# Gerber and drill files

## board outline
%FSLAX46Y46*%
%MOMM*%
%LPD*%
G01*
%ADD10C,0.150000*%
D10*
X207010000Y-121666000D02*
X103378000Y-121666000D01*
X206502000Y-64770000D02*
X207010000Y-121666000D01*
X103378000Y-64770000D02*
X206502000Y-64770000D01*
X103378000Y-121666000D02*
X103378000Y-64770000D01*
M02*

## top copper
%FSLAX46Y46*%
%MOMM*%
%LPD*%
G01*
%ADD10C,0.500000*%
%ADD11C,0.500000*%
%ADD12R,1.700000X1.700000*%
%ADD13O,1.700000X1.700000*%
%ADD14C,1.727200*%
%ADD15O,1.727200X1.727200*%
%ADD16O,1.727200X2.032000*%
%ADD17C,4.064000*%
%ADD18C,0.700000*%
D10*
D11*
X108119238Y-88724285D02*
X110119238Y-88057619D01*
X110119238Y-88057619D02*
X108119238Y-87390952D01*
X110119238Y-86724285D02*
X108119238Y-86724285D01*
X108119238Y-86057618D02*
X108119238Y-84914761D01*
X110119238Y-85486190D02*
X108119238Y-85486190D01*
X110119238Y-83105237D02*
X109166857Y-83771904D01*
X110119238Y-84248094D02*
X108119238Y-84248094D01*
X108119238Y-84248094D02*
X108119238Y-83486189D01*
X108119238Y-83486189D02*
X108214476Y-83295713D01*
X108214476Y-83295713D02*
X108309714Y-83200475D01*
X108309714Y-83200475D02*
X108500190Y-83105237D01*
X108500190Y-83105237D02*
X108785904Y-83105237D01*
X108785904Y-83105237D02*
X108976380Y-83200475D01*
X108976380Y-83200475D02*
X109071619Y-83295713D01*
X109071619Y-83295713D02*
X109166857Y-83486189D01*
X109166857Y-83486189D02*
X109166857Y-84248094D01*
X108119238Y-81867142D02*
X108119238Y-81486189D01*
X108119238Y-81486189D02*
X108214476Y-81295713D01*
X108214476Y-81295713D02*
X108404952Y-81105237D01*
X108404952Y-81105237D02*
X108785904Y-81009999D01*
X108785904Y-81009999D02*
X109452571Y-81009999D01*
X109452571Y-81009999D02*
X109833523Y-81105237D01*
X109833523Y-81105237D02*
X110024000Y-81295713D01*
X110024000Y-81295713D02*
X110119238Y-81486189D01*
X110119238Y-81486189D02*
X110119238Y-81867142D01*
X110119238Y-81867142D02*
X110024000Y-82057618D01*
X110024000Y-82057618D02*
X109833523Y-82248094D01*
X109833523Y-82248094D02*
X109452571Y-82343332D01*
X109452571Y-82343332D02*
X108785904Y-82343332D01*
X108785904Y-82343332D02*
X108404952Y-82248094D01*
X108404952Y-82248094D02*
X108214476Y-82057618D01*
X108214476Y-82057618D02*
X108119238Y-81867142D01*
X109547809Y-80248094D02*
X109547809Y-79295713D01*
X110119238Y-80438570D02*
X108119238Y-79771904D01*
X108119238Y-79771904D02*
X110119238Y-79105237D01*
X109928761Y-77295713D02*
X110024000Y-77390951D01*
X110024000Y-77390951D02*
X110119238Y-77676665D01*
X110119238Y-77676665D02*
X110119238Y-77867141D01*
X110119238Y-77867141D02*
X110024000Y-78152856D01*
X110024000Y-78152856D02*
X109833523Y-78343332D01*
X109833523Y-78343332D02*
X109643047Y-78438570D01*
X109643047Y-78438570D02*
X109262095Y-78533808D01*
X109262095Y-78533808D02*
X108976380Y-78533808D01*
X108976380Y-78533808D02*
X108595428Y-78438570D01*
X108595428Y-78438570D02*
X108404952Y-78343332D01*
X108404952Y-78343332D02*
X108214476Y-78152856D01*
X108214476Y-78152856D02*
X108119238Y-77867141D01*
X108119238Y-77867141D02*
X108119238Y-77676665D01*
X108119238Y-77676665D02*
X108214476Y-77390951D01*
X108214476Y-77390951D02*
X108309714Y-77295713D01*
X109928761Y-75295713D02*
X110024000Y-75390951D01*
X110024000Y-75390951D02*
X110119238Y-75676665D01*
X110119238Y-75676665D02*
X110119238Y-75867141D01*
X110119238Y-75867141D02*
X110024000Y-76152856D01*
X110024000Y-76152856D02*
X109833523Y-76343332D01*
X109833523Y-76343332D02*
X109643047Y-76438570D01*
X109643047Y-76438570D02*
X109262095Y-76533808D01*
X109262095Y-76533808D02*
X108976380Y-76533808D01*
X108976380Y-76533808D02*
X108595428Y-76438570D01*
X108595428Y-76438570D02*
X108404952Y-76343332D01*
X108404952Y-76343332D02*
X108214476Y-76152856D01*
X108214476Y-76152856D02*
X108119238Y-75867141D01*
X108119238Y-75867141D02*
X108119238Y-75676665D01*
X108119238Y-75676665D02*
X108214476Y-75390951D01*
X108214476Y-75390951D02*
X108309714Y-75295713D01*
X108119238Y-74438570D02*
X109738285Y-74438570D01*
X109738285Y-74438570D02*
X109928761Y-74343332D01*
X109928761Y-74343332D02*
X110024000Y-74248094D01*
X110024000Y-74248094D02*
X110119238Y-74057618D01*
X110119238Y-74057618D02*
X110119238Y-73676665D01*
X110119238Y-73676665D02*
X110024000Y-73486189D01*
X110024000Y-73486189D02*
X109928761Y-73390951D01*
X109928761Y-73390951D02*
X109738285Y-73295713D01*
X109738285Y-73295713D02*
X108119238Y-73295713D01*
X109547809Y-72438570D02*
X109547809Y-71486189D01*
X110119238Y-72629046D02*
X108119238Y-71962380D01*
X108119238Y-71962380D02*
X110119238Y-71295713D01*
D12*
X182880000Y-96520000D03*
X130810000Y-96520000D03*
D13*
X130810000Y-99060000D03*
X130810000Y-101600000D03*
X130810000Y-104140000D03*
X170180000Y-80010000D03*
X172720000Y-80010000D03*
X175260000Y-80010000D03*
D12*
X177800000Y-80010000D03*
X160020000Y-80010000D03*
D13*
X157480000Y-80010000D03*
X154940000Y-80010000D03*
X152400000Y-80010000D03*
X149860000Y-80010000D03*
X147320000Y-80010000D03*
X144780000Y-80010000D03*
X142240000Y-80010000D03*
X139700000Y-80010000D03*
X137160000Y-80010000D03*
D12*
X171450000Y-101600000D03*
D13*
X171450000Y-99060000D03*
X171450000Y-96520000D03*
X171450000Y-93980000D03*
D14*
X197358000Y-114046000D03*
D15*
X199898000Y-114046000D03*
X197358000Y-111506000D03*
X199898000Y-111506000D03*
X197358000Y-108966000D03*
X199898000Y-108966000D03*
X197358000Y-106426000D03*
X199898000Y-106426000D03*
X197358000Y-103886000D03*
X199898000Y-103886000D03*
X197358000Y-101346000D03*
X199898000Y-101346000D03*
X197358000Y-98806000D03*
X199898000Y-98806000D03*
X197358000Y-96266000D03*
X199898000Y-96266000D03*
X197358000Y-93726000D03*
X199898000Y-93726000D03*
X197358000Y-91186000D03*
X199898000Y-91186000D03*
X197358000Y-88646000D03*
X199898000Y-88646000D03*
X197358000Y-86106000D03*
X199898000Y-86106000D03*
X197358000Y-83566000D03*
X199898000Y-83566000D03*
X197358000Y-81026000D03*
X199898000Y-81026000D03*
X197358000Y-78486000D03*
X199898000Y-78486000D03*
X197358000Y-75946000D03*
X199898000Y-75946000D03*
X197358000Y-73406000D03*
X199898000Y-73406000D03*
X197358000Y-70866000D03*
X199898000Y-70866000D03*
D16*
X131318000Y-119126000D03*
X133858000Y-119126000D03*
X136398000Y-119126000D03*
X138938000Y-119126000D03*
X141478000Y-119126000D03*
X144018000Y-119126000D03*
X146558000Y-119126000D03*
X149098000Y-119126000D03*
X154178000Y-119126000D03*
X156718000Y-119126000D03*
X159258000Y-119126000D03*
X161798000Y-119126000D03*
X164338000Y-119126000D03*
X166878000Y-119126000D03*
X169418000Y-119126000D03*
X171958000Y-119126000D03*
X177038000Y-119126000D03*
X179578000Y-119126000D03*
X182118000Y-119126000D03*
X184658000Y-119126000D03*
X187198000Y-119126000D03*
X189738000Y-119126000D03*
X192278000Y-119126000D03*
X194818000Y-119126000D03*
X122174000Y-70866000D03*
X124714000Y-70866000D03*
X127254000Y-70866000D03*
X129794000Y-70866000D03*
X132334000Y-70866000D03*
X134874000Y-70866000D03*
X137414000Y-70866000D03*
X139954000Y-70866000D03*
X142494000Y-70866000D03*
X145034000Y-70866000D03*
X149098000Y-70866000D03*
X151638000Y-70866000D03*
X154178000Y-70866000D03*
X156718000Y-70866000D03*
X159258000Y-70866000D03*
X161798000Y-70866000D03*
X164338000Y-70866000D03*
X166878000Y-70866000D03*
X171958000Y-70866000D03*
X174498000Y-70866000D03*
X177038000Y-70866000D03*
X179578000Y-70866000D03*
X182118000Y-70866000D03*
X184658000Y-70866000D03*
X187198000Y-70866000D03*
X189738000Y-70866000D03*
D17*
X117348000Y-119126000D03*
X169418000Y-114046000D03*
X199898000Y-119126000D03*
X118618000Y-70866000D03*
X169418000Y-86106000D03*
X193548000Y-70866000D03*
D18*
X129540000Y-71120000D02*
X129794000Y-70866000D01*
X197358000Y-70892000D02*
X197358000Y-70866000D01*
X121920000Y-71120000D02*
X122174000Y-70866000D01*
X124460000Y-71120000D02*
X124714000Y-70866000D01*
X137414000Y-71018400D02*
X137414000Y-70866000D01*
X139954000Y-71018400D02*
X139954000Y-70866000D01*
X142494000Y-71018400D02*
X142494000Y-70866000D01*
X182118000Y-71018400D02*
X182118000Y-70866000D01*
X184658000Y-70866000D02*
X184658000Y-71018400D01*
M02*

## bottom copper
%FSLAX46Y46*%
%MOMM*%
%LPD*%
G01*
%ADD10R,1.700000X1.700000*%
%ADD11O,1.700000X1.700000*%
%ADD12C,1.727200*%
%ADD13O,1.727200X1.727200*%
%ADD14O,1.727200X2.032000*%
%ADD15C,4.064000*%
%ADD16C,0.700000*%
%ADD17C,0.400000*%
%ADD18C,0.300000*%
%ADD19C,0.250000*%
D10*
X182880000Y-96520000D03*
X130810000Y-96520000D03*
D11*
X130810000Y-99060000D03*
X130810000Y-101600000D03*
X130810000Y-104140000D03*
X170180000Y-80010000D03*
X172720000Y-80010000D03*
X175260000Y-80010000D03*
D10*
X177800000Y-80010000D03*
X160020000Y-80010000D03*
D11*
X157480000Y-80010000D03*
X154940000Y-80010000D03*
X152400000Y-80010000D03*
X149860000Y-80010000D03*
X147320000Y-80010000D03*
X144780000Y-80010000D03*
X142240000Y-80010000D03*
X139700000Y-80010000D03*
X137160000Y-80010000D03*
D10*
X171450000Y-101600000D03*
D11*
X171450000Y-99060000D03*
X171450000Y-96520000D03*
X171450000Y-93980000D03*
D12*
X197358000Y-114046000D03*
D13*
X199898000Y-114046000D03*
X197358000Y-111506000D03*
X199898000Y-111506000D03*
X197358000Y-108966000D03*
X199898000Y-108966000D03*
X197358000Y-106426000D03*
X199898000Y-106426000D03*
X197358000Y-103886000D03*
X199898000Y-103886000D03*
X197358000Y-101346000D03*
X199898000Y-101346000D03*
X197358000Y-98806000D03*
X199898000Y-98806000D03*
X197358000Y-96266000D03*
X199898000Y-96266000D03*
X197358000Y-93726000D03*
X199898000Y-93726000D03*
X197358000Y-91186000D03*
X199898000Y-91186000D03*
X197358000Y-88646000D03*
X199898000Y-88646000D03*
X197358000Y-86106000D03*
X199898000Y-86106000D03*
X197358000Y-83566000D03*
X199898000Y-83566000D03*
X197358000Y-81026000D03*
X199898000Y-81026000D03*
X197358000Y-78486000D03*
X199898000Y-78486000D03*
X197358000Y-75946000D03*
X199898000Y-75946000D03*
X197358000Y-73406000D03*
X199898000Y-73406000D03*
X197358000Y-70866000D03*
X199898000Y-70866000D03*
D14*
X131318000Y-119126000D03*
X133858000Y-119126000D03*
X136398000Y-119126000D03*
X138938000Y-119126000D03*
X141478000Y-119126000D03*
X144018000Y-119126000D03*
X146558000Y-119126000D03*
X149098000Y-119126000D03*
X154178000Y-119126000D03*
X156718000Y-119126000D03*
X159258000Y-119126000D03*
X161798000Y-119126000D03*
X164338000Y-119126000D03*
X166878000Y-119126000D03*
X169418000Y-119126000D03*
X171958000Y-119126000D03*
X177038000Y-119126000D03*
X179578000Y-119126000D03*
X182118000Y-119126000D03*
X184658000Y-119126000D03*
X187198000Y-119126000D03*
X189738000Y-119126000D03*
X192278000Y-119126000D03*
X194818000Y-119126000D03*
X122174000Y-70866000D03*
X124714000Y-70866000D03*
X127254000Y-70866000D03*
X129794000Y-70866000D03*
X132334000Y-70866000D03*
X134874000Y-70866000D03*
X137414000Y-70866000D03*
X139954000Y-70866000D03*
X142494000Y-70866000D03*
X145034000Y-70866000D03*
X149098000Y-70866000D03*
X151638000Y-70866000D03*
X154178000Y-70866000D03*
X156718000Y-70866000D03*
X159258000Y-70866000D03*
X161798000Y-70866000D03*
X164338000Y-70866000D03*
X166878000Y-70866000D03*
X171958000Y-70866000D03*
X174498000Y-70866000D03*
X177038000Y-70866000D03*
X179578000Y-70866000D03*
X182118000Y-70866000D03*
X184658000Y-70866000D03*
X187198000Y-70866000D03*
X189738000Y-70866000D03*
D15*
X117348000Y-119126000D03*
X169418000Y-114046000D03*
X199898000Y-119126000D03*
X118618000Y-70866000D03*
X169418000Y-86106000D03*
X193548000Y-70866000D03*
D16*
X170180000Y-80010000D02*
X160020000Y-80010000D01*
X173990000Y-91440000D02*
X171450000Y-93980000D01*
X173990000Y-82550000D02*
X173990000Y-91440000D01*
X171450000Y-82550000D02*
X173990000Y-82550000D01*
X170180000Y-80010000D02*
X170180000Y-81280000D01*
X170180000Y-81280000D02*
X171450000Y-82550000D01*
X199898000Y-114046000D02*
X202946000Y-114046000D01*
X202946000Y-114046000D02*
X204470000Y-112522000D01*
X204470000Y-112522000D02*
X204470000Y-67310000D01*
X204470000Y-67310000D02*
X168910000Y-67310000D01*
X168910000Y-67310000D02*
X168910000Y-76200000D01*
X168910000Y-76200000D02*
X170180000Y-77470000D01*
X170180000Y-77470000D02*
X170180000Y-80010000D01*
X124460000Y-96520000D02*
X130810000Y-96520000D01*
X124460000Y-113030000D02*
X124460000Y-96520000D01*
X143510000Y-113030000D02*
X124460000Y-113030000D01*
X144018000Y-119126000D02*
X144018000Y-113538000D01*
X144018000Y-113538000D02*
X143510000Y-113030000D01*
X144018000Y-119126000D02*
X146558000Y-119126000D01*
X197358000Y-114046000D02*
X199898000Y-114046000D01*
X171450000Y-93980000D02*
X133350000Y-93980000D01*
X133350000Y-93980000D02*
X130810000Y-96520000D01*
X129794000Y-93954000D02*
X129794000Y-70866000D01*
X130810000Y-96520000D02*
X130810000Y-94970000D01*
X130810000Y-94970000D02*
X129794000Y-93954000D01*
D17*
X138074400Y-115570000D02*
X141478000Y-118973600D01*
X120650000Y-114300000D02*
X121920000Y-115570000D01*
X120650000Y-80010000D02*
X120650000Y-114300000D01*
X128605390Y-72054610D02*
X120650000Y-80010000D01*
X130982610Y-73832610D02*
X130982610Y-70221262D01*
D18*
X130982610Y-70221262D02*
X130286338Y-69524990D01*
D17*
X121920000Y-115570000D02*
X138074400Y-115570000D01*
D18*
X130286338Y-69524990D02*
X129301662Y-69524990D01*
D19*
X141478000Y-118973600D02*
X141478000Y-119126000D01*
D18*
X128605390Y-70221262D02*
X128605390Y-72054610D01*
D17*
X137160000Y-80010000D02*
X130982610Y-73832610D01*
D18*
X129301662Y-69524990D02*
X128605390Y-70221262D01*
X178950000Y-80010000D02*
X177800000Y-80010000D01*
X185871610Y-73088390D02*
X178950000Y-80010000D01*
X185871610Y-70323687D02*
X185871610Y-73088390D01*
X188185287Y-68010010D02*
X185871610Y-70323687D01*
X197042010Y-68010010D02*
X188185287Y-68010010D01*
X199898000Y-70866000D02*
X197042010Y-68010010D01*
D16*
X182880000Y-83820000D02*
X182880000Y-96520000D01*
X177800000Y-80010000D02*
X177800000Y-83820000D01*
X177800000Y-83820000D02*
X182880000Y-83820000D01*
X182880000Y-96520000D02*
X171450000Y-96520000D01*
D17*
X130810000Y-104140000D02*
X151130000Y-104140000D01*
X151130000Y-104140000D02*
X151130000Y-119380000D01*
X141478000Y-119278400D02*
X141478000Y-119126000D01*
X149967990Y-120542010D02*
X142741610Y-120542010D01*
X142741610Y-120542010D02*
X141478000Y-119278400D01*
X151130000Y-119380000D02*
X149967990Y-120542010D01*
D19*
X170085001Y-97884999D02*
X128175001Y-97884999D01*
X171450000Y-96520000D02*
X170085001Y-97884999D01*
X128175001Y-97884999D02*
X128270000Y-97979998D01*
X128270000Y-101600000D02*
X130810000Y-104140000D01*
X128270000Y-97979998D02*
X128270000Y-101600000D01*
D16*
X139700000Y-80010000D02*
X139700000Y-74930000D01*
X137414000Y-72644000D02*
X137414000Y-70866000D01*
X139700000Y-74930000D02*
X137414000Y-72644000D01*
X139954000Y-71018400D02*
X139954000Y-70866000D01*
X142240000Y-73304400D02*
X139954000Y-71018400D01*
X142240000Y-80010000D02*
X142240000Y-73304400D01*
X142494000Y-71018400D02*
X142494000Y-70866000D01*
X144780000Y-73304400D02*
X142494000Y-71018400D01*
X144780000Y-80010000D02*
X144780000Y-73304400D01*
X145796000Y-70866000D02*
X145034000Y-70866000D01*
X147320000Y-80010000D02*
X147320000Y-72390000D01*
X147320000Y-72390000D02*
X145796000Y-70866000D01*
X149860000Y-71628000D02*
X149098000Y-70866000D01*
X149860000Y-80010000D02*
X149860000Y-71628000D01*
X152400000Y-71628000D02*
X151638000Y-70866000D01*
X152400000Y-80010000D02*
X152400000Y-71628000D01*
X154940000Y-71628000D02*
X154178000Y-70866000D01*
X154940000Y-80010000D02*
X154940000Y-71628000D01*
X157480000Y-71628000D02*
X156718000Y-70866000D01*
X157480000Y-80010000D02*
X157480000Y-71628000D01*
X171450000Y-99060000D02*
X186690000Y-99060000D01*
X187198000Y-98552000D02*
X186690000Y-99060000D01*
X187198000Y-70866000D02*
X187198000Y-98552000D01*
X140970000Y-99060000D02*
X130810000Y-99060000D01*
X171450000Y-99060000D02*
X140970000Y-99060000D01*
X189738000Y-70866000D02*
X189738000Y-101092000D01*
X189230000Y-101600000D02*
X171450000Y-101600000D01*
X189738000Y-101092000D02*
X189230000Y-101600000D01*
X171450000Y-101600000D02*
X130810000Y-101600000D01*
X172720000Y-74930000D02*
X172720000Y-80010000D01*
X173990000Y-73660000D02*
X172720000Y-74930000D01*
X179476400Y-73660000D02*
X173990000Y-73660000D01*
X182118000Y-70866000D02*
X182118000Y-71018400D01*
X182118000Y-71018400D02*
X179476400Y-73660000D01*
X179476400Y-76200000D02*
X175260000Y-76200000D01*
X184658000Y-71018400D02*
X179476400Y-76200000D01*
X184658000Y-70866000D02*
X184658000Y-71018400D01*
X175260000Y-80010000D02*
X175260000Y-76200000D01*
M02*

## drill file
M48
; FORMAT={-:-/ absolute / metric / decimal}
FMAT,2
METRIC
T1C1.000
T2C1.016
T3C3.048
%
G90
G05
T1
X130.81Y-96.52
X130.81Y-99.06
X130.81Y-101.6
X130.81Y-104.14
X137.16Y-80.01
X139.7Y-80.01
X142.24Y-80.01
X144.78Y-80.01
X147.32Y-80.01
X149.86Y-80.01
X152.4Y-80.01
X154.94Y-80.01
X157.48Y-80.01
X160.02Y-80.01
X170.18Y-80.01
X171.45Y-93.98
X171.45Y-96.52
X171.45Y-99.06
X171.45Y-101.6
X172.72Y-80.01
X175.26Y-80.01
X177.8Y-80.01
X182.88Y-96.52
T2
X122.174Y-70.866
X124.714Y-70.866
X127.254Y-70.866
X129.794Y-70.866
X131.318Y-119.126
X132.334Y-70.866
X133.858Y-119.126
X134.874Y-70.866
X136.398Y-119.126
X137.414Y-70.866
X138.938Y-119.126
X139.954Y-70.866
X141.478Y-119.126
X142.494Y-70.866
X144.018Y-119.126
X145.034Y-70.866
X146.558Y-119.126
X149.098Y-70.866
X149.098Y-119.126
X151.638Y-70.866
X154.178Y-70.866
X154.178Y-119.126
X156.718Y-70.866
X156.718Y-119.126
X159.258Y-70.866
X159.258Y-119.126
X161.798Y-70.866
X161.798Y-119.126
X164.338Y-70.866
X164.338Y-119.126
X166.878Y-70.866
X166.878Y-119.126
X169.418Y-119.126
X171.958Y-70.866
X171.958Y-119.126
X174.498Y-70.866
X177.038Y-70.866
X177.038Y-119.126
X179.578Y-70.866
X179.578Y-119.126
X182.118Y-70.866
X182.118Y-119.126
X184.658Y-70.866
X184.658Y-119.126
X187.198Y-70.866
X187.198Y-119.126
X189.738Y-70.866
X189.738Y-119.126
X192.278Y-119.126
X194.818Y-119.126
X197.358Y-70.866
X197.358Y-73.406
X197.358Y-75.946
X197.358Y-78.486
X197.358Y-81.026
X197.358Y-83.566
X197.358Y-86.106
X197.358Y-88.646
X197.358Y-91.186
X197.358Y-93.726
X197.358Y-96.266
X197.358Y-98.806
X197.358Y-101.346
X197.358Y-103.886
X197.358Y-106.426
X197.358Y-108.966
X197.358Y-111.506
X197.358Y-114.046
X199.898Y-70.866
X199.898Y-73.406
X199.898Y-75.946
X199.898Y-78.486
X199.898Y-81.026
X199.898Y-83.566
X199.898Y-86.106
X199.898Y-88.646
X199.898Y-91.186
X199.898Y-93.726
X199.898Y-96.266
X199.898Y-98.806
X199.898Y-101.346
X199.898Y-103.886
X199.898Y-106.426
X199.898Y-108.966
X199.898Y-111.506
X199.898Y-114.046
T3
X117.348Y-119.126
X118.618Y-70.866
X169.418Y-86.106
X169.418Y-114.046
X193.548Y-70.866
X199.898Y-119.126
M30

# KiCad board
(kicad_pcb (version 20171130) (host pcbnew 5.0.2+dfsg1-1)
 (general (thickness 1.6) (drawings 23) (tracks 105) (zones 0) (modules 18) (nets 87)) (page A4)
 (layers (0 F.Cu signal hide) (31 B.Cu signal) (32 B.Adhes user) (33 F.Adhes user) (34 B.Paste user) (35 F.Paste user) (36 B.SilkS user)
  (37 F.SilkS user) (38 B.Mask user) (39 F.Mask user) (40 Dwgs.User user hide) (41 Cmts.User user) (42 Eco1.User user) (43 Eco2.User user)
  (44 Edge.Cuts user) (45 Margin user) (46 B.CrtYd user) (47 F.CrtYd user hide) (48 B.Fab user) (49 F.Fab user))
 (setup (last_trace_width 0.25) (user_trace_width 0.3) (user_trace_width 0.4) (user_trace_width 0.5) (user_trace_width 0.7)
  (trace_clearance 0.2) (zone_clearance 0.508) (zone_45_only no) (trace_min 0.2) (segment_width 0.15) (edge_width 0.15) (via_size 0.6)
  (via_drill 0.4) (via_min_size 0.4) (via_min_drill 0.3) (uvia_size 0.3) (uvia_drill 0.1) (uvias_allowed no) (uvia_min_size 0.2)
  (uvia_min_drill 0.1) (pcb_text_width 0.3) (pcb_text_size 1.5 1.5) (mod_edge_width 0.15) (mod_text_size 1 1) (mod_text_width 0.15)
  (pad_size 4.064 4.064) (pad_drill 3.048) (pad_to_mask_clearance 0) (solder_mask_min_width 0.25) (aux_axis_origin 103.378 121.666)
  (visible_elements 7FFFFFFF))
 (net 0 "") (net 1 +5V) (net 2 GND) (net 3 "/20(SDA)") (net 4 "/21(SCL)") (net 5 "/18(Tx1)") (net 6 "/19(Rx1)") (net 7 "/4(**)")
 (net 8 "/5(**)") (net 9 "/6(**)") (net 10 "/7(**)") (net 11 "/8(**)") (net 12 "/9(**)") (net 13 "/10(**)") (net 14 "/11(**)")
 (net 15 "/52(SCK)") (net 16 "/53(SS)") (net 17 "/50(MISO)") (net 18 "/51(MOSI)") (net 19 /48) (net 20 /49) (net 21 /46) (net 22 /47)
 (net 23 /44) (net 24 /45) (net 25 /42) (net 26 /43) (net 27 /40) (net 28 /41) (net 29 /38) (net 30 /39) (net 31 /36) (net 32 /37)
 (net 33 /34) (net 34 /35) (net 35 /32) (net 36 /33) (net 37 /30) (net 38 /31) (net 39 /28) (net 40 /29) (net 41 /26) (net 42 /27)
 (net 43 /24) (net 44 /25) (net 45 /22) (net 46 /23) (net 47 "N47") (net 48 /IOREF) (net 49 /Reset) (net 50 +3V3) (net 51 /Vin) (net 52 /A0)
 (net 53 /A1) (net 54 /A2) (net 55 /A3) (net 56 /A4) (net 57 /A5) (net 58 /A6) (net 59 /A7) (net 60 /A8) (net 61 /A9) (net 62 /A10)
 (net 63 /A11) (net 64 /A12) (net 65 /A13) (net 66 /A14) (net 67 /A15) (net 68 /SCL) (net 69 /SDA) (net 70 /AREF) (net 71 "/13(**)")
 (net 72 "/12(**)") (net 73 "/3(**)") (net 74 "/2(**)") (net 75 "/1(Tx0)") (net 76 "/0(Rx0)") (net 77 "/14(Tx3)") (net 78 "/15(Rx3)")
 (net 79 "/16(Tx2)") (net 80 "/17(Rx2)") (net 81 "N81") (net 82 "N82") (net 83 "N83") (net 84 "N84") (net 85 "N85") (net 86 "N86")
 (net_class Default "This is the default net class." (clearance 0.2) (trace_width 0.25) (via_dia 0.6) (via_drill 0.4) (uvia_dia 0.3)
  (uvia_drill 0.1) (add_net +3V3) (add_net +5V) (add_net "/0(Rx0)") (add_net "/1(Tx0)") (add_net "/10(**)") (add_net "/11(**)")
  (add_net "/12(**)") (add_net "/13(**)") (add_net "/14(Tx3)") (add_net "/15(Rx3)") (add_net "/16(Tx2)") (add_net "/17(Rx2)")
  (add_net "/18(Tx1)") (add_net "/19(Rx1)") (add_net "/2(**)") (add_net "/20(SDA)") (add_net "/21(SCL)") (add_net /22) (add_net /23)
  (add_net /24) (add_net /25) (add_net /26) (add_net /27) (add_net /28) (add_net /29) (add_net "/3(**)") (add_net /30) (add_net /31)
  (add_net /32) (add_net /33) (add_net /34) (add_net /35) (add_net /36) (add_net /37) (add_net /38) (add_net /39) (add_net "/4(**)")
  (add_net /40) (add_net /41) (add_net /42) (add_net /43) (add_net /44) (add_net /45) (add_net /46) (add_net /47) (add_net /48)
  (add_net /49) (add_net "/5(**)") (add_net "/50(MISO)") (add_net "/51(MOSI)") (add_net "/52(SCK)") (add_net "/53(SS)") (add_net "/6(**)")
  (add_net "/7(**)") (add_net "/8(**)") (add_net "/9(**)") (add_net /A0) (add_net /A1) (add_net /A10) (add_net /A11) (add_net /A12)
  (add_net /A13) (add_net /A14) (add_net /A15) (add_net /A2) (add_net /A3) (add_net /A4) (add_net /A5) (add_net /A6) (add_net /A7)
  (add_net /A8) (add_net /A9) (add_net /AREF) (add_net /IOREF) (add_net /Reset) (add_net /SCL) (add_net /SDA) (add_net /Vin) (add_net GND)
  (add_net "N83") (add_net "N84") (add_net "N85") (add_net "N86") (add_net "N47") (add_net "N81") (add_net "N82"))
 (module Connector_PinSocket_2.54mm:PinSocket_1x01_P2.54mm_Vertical (layer F.Cu) (at 182.88 96.52)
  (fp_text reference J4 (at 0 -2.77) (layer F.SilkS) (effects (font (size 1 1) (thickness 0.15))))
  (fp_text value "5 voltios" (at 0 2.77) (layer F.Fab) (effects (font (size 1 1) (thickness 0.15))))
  (pad 1 thru_hole rect (at 0 0) (size 1.7 1.7) (drill 1) (layers *.Cu *.Mask) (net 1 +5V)))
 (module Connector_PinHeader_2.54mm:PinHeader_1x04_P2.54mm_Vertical (layer F.Cu) (at 130.81 96.52)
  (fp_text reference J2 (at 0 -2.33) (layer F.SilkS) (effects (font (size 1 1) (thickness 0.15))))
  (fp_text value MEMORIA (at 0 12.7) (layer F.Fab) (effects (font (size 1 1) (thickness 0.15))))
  (pad 1 thru_hole rect (at 0 0) (size 1.7 1.7) (drill 1) (layers *.Cu *.Mask) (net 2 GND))
  (pad 2 thru_hole oval (at 0 2.54) (size 1.7 1.7) (drill 1) (layers *.Cu *.Mask) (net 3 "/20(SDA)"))
  (pad 3 thru_hole oval (at 0 5.08) (size 1.7 1.7) (drill 1) (layers *.Cu *.Mask) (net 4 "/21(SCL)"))
  (pad 4 thru_hole oval (at 0 7.62) (size 1.7 1.7) (drill 1) (layers *.Cu *.Mask) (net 1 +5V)))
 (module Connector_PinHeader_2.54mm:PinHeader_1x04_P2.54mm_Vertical (layer F.Cu) (at 177.8 80.01 270)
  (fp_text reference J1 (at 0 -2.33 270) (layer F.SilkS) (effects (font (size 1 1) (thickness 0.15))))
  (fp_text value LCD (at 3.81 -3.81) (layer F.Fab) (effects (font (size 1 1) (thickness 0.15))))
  (pad 4 thru_hole oval (at 0 7.62 270) (size 1.7 1.7) (drill 1) (layers *.Cu *.Mask) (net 2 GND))
  (pad 3 thru_hole oval (at 0 5.08 270) (size 1.7 1.7) (drill 1) (layers *.Cu *.Mask) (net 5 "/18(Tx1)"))
  (pad 2 thru_hole oval (at 0 2.54 270) (size 1.7 1.7) (drill 1) (layers *.Cu *.Mask) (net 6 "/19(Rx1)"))
  (pad 1 thru_hole rect (at 0 0 270) (size 1.7 1.7) (drill 1) (layers *.Cu *.Mask) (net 1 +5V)))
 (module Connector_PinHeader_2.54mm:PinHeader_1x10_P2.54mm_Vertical (layer F.Cu) (at 160.02 80.01 270)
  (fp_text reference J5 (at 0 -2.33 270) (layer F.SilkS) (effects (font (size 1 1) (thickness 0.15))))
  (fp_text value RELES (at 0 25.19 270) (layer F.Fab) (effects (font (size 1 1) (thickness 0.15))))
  (pad 1 thru_hole rect (at 0 0 270) (size 1.7 1.7) (drill 1) (layers *.Cu *.Mask) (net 2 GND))
  (pad 2 thru_hole oval (at 0 2.54 270) (size 1.7 1.7) (drill 1) (layers *.Cu *.Mask) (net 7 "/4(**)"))
  (pad 3 thru_hole oval (at 0 5.08 270) (size 1.7 1.7) (drill 1) (layers *.Cu *.Mask) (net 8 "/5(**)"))
  (pad 4 thru_hole oval (at 0 7.62 270) (size 1.7 1.7) (drill 1) (layers *.Cu *.Mask) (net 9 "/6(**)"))
  (pad 5 thru_hole oval (at 0 10.16 270) (size 1.7 1.7) (drill 1) (layers *.Cu *.Mask) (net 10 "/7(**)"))
  (pad 6 thru_hole oval (at 0 12.7 270) (size 1.7 1.7) (drill 1) (layers *.Cu *.Mask) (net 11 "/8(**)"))
  (pad 7 thru_hole oval (at 0 15.24 270) (size 1.7 1.7) (drill 1) (layers *.Cu *.Mask) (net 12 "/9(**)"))
  (pad 8 thru_hole oval (at 0 17.78 270) (size 1.7 1.7) (drill 1) (layers *.Cu *.Mask) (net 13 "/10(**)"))
  (pad 9 thru_hole oval (at 0 20.32 270) (size 1.7 1.7) (drill 1) (layers *.Cu *.Mask) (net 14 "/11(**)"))
  (pad 10 thru_hole oval (at 0 22.86 270) (size 1.7 1.7) (drill 1) (layers *.Cu *.Mask) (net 1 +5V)))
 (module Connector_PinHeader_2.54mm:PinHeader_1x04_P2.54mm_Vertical (layer F.Cu) (at 171.45 101.6 180)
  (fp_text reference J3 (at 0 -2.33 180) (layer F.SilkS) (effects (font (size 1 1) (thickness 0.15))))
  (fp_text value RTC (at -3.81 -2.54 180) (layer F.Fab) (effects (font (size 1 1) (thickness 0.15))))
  (pad 1 thru_hole rect (at 0 0 180) (size 1.7 1.7) (drill 1) (layers *.Cu *.Mask) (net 4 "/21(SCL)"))
  (pad 2 thru_hole oval (at 0 2.54 180) (size 1.7 1.7) (drill 1) (layers *.Cu *.Mask) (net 3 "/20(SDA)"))
  (pad 3 thru_hole oval (at 0 5.08 180) (size 1.7 1.7) (drill 1) (layers *.Cu *.Mask) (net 1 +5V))
  (pad 4 thru_hole oval (at 0 7.62 180) (size 1.7 1.7) (drill 1) (layers *.Cu *.Mask) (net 2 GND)))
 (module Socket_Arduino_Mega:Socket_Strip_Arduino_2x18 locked (layer F.Cu) (at 197.358 114.046 90)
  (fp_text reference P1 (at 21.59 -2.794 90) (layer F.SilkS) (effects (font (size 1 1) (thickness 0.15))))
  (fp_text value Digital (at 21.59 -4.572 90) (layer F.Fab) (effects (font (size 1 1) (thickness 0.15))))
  (pad 1 thru_hole circle (at 0 0 90) (size 1.7272 1.7272) (drill 1.016) (layers *.Cu *.Mask F.SilkS) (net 2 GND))
  (pad 2 thru_hole oval (at 0 2.54 90) (size 1.7272 1.7272) (drill 1.016) (layers *.Cu *.Mask F.SilkS) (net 2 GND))
  (pad 3 thru_hole oval (at 2.54 0 90) (size 1.7272 1.7272) (drill 1.016) (layers *.Cu *.Mask F.SilkS) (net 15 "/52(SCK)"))
  (pad 4 thru_hole oval (at 2.54 2.54 90) (size 1.7272 1.7272) (drill 1.016) (layers *.Cu *.Mask F.SilkS) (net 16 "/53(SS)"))
  (pad 5 thru_hole oval (at 5.08 0 90) (size 1.7272 1.7272) (drill 1.016) (layers *.Cu *.Mask F.SilkS) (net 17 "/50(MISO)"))
  (pad 6 thru_hole oval (at 5.08 2.54 90) (size 1.7272 1.7272) (drill 1.016) (layers *.Cu *.Mask F.SilkS) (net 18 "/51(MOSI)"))
  (pad 7 thru_hole oval (at 7.62 0 90) (size 1.7272 1.7272) (drill 1.016) (layers *.Cu *.Mask F.SilkS) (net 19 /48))
  (pad 8 thru_hole oval (at 7.62 2.54 90) (size 1.7272 1.7272) (drill 1.016) (layers *.Cu *.Mask F.SilkS) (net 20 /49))
  (pad 9 thru_hole oval (at 10.16 0 90) (size 1.7272 1.7272) (drill 1.016) (layers *.Cu *.Mask F.SilkS) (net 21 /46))
  (pad 10 thru_hole oval (at 10.16 2.54 90) (size 1.7272 1.7272) (drill 1.016) (layers *.Cu *.Mask F.SilkS) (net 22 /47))
  (pad 11 thru_hole oval (at 12.7 0 90) (size 1.7272 1.7272) (drill 1.016) (layers *.Cu *.Mask F.SilkS) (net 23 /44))
  (pad 12 thru_hole oval (at 12.7 2.54 90) (size 1.7272 1.7272) (drill 1.016) (layers *.Cu *.Mask F.SilkS) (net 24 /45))
  (pad 13 thru_hole oval (at 15.24 0 90) (size 1.7272 1.7272) (drill 1.016) (layers *.Cu *.Mask F.SilkS) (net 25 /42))
  (pad 14 thru_hole oval (at 15.24 2.54 90) (size 1.7272 1.7272) (drill 1.016) (layers *.Cu *.Mask F.SilkS) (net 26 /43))
  (pad 15 thru_hole oval (at 17.78 0 90) (size 1.7272 1.7272) (drill 1.016) (layers *.Cu *.Mask F.SilkS) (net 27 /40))
  (pad 16 thru_hole oval (at 17.78 2.54 90) (size 1.7272 1.7272) (drill 1.016) (layers *.Cu *.Mask F.SilkS) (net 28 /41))
  (pad 17 thru_hole oval (at 20.32 0 90) (size 1.7272 1.7272) (drill 1.016) (layers *.Cu *.Mask F.SilkS) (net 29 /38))
  (pad 18 thru_hole oval (at 20.32 2.54 90) (size 1.7272 1.7272) (drill 1.016) (layers *.Cu *.Mask F.SilkS) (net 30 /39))
  (pad 19 thru_hole oval (at 22.86 0 90) (size 1.7272 1.7272) (drill 1.016) (layers *.Cu *.Mask F.SilkS) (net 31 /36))
  (pad 20 thru_hole oval (at 22.86 2.54 90) (size 1.7272 1.7272) (drill 1.016) (layers *.Cu *.Mask F.SilkS) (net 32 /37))
  (pad 21 thru_hole oval (at 25.4 0 90) (size 1.7272 1.7272) (drill 1.016) (layers *.Cu *.Mask F.SilkS) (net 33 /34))
  (pad 22 thru_hole oval (at 25.4 2.54 90) (size 1.7272 1.7272) (drill 1.016) (layers *.Cu *.Mask F.SilkS) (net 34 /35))
  (pad 23 thru_hole oval (at 27.94 0 90) (size 1.7272 1.7272) (drill 1.016) (layers *.Cu *.Mask F.SilkS) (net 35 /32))
  (pad 24 thru_hole oval (at 27.94 2.54 90) (size 1.7272 1.7272) (drill 1.016) (layers *.Cu *.Mask F.SilkS) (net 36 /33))
  (pad 25 thru_hole oval (at 30.48 0 90) (size 1.7272 1.7272) (drill 1.016) (layers *.Cu *.Mask F.SilkS) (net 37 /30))
  (pad 26 thru_hole oval (at 30.48 2.54 90) (size 1.7272 1.7272) (drill 1.016) (layers *.Cu *.Mask F.SilkS) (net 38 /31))
  (pad 27 thru_hole oval (at 33.02 0 90) (size 1.7272 1.7272) (drill 1.016) (layers *.Cu *.Mask F.SilkS) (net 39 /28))
  (pad 28 thru_hole oval (at 33.02 2.54 90) (size 1.7272 1.7272) (drill 1.016) (layers *.Cu *.Mask F.SilkS) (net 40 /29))
  (pad 29 thru_hole oval (at 35.56 0 90) (size 1.7272 1.7272) (drill 1.016) (layers *.Cu *.Mask F.SilkS) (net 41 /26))
  (pad 30 thru_hole oval (at 35.56 2.54 90) (size 1.7272 1.7272) (drill 1.016) (layers *.Cu *.Mask F.SilkS) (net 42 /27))
  (pad 31 thru_hole oval (at 38.1 0 90) (size 1.7272 1.7272) (drill 1.016) (layers *.Cu *.Mask F.SilkS) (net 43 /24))
  (pad 32 thru_hole oval (at 38.1 2.54 90) (size 1.7272 1.7272) (drill 1.016) (layers *.Cu *.Mask F.SilkS) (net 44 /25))
  (pad 33 thru_hole oval (at 40.64 0 90) (size 1.7272 1.7272) (drill 1.016) (layers *.Cu *.Mask F.SilkS) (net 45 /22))
  (pad 34 thru_hole oval (at 40.64 2.54 90) (size 1.7272 1.7272) (drill 1.016) (layers *.Cu *.Mask F.SilkS) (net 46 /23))
  (pad 35 thru_hole oval (at 43.18 0 90) (size 1.7272 1.7272) (drill 1.016) (layers *.Cu *.Mask F.SilkS) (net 1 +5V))
  (pad 36 thru_hole oval (at 43.18 2.54 90) (size 1.7272 1.7272) (drill 1.016) (layers *.Cu *.Mask F.SilkS) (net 1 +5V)))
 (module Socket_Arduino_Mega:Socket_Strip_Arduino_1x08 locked (layer F.Cu) (at 131.318 119.126)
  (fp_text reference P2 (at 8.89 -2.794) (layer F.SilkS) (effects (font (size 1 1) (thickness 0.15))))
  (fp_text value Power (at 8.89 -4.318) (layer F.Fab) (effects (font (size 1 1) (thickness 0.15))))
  (pad 1 thru_hole oval (at 0 0) (size 1.7272 2.032) (drill 1.016) (layers *.Cu *.Mask F.SilkS) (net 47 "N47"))
  (pad 2 thru_hole oval (at 2.54 0) (size 1.7272 2.032) (drill 1.016) (layers *.Cu *.Mask F.SilkS) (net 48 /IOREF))
  (pad 3 thru_hole oval (at 5.08 0) (size 1.7272 2.032) (drill 1.016) (layers *.Cu *.Mask F.SilkS) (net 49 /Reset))
  (pad 4 thru_hole oval (at 7.62 0) (size 1.7272 2.032) (drill 1.016) (layers *.Cu *.Mask F.SilkS) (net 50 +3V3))
  (pad 5 thru_hole oval (at 10.16 0) (size 1.7272 2.032) (drill 1.016) (layers *.Cu *.Mask F.SilkS) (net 1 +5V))
  (pad 6 thru_hole oval (at 12.7 0) (size 1.7272 2.032) (drill 1.016) (layers *.Cu *.Mask F.SilkS) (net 2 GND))
  (pad 7 thru_hole oval (at 15.24 0) (size 1.7272 2.032) (drill 1.016) (layers *.Cu *.Mask F.SilkS) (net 2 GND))
  (pad 8 thru_hole oval (at 17.78 0) (size 1.7272 2.032) (drill 1.016) (layers *.Cu *.Mask F.SilkS) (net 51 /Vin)))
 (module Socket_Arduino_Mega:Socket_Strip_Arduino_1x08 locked (layer F.Cu) (at 154.178 119.126)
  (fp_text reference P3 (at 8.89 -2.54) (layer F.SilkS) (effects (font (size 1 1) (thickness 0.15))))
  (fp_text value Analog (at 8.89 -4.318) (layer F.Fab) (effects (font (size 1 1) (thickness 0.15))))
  (pad 1 thru_hole oval (at 0 0) (size 1.7272 2.032) (drill 1.016) (layers *.Cu *.Mask F.SilkS) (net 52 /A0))
  (pad 2 thru_hole oval (at 2.54 0) (size 1.7272 2.032) (drill 1.016) (layers *.Cu *.Mask F.SilkS) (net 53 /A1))
  (pad 3 thru_hole oval (at 5.08 0) (size 1.7272 2.032) (drill 1.016) (layers *.Cu *.Mask F.SilkS) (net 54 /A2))
  (pad 4 thru_hole oval (at 7.62 0) (size 1.7272 2.032) (drill 1.016) (layers *.Cu *.Mask F.SilkS) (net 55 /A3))
  (pad 5 thru_hole oval (at 10.16 0) (size 1.7272 2.032) (drill 1.016) (layers *.Cu *.Mask F.SilkS) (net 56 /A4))
  (pad 6 thru_hole oval (at 12.7 0) (size 1.7272 2.032) (drill 1.016) (layers *.Cu *.Mask F.SilkS) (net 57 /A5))
  (pad 7 thru_hole oval (at 15.24 0) (size 1.7272 2.032) (drill 1.016) (layers *.Cu *.Mask F.SilkS) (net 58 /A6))
  (pad 8 thru_hole oval (at 17.78 0) (size 1.7272 2.032) (drill 1.016) (layers *.Cu *.Mask F.SilkS) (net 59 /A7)))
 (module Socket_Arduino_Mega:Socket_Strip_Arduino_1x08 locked (layer F.Cu) (at 177.038 119.126)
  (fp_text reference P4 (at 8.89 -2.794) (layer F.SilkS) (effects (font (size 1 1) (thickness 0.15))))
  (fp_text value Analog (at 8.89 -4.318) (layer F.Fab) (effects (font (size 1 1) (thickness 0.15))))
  (pad 1 thru_hole oval (at 0 0) (size 1.7272 2.032) (drill 1.016) (layers *.Cu *.Mask F.SilkS) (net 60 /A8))
  (pad 2 thru_hole oval (at 2.54 0) (size 1.7272 2.032) (drill 1.016) (layers *.Cu *.Mask F.SilkS) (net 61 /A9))
  (pad 3 thru_hole oval (at 5.08 0) (size 1.7272 2.032) (drill 1.016) (layers *.Cu *.Mask F.SilkS) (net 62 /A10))
  (pad 4 thru_hole oval (at 7.62 0) (size 1.7272 2.032) (drill 1.016) (layers *.Cu *.Mask F.SilkS) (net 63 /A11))
  (pad 5 thru_hole oval (at 10.16 0) (size 1.7272 2.032) (drill 1.016) (layers *.Cu *.Mask F.SilkS) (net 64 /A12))
  (pad 6 thru_hole oval (at 12.7 0) (size 1.7272 2.032) (drill 1.016) (layers *.Cu *.Mask F.SilkS) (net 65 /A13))
  (pad 7 thru_hole oval (at 15.24 0) (size 1.7272 2.032) (drill 1.016) (layers *.Cu *.Mask F.SilkS) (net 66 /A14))
  (pad 8 thru_hole oval (at 17.78 0) (size 1.7272 2.032) (drill 1.016) (layers *.Cu *.Mask F.SilkS) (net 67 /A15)))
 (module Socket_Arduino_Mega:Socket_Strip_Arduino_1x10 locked (layer F.Cu) (at 122.174 70.866)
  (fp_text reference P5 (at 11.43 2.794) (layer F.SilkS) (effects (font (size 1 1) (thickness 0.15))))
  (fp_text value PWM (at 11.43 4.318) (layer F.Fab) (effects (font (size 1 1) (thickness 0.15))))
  (pad 1 thru_hole oval (at 0 0) (size 1.7272 2.032) (drill 1.016) (layers *.Cu *.Mask F.SilkS) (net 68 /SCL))
  (pad 2 thru_hole oval (at 2.54 0) (size 1.7272 2.032) (drill 1.016) (layers *.Cu *.Mask F.SilkS) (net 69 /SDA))
  (pad 3 thru_hole oval (at 5.08 0) (size 1.7272 2.032) (drill 1.016) (layers *.Cu *.Mask F.SilkS) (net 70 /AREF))
  (pad 4 thru_hole oval (at 7.62 0) (size 1.7272 2.032) (drill 1.016) (layers *.Cu *.Mask F.SilkS) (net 2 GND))
  (pad 5 thru_hole oval (at 10.16 0) (size 1.7272 2.032) (drill 1.016) (layers *.Cu *.Mask F.SilkS) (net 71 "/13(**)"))
  (pad 6 thru_hole oval (at 12.7 0) (size 1.7272 2.032) (drill 1.016) (layers *.Cu *.Mask F.SilkS) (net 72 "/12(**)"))
  (pad 7 thru_hole oval (at 15.24 0) (size 1.7272 2.032) (drill 1.016) (layers *.Cu *.Mask F.SilkS) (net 14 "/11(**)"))
  (pad 8 thru_hole oval (at 17.78 0) (size 1.7272 2.032) (drill 1.016) (layers *.Cu *.Mask F.SilkS) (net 13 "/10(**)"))
  (pad 9 thru_hole oval (at 20.32 0) (size 1.7272 2.032) (drill 1.016) (layers *.Cu *.Mask F.SilkS) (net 12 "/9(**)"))
  (pad 10 thru_hole oval (at 22.86 0) (size 1.7272 2.032) (drill 1.016) (layers *.Cu *.Mask F.SilkS) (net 11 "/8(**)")))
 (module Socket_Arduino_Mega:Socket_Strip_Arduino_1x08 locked (layer F.Cu) (at 149.098 70.866)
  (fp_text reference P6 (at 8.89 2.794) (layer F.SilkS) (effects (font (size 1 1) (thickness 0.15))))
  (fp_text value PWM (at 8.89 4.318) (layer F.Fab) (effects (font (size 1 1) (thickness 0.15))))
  (pad 1 thru_hole oval (at 0 0) (size 1.7272 2.032) (drill 1.016) (layers *.Cu *.Mask F.SilkS) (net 10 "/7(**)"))
  (pad 2 thru_hole oval (at 2.54 0) (size 1.7272 2.032) (drill 1.016) (layers *.Cu *.Mask F.SilkS) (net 9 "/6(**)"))
  (pad 3 thru_hole oval (at 5.08 0) (size 1.7272 2.032) (drill 1.016) (layers *.Cu *.Mask F.SilkS) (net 8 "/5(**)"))
  (pad 4 thru_hole oval (at 7.62 0) (size 1.7272 2.032) (drill 1.016) (layers *.Cu *.Mask F.SilkS) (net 7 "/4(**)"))
  (pad 5 thru_hole oval (at 10.16 0) (size 1.7272 2.032) (drill 1.016) (layers *.Cu *.Mask F.SilkS) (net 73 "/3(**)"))
  (pad 6 thru_hole oval (at 12.7 0) (size 1.7272 2.032) (drill 1.016) (layers *.Cu *.Mask F.SilkS) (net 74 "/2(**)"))
  (pad 7 thru_hole oval (at 15.24 0) (size 1.7272 2.032) (drill 1.016) (layers *.Cu *.Mask F.SilkS) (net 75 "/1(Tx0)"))
  (pad 8 thru_hole oval (at 17.78 0) (size 1.7272 2.032) (drill 1.016) (layers *.Cu *.Mask F.SilkS) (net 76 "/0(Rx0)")))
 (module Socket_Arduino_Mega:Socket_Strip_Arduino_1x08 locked (layer F.Cu) (at 171.958 70.866)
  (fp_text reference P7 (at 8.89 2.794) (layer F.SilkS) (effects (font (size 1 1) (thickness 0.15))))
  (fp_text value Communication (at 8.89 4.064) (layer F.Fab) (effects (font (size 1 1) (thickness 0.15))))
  (pad 1 thru_hole oval (at 0 0) (size 1.7272 2.032) (drill 1.016) (layers *.Cu *.Mask F.SilkS) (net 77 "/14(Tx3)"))
  (pad 2 thru_hole oval (at 2.54 0) (size 1.7272 2.032) (drill 1.016) (layers *.Cu *.Mask F.SilkS) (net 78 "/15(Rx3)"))
  (pad 3 thru_hole oval (at 5.08 0) (size 1.7272 2.032) (drill 1.016) (layers *.Cu *.Mask F.SilkS) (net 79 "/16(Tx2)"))
  (pad 4 thru_hole oval (at 7.62 0) (size 1.7272 2.032) (drill 1.016) (layers *.Cu *.Mask F.SilkS) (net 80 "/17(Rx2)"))
  (pad 5 thru_hole oval (at 10.16 0) (size 1.7272 2.032) (drill 1.016) (layers *.Cu *.Mask F.SilkS) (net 5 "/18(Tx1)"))
  (pad 6 thru_hole oval (at 12.7 0) (size 1.7272 2.032) (drill 1.016) (layers *.Cu *.Mask F.SilkS) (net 6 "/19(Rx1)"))
  (pad 7 thru_hole oval (at 15.24 0) (size 1.7272 2.032) (drill 1.016) (layers *.Cu *.Mask F.SilkS) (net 3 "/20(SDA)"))
  (pad 8 thru_hole oval (at 17.78 0) (size 1.7272 2.032) (drill 1.016) (layers *.Cu *.Mask F.SilkS) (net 4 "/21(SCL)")))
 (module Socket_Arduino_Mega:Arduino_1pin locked (layer F.Cu) (at 117.348 119.126)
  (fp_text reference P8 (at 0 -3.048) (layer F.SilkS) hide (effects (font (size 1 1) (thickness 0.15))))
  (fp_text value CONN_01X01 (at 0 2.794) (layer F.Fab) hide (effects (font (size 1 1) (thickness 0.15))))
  (pad 1 thru_hole circle (at 0 0) (size 4.064 4.064) (drill 3.048) (layers *.Cu *.Mask F.SilkS) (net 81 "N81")))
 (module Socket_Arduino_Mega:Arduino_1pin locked (layer F.Cu) (at 169.418 114.046)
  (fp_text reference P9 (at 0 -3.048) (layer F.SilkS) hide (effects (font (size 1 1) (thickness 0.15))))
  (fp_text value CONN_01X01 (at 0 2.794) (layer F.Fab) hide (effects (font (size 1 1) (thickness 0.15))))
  (pad 1 thru_hole circle (at 0 0) (size 4.064 4.064) (drill 3.048) (layers *.Cu *.Mask F.SilkS) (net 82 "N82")))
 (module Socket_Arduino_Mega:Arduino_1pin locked (layer F.Cu) (at 199.898 119.126)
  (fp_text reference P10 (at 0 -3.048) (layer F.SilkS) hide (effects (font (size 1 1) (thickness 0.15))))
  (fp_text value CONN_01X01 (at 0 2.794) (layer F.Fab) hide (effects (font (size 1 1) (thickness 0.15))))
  (pad 1 thru_hole circle (at 0 0) (size 4.064 4.064) (drill 3.048) (layers *.Cu *.Mask F.SilkS) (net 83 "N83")))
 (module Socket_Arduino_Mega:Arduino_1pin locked (layer F.Cu) (at 118.618 70.866)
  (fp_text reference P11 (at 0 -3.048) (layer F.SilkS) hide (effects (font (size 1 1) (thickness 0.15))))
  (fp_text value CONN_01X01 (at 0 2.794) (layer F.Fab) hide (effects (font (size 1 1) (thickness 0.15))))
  (pad 1 thru_hole circle (at 0 0) (size 4.064 4.064) (drill 3.048) (layers *.Cu *.Mask F.SilkS) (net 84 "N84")))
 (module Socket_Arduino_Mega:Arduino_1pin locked (layer F.Cu) (at 169.418 86.106)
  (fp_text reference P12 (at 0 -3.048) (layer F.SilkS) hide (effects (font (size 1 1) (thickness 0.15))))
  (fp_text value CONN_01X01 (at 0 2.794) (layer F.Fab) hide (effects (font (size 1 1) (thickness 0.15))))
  (pad 1 thru_hole circle (at 0 0) (size 4.064 4.064) (drill 3.048) (layers *.Cu *.Mask F.SilkS) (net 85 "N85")))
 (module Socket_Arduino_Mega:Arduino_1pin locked (layer F.Cu) (at 193.548 70.866)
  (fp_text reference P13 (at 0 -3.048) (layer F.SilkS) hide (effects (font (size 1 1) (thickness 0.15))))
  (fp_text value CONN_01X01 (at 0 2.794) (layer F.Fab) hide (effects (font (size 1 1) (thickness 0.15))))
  (pad 1 thru_hole circle (at 0 0) (size 4.064 4.064) (drill 3.048) (layers *.Cu *.Mask F.SilkS) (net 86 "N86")))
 (gr_line (start 207.01 121.666) (end 103.378 121.666) (angle 90) (layer Edge.Cuts) (width 0.15))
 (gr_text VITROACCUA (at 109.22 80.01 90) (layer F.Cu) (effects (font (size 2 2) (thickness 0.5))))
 (gr_line (start 206.502 64.77) (end 207.01 121.666) (angle 90) (layer Edge.Cuts) (width 0.15))
 (gr_line (start 103.378 64.77) (end 206.502 64.77) (angle 90) (layer Edge.Cuts) (width 0.15))
 (gr_line (start 103.378 121.666) (end 103.378 64.77) (angle 90) (layer Edge.Cuts) (width 0.15))
 (segment (start 129.54 71.12) (end 129.794 70.866) (width 0.7) (layer F.Cu) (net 2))
 (segment (start 170.18 80.01) (end 160.02 80.01) (width 0.7) (layer B.Cu) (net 2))
 (segment (start 173.99 91.44) (end 171.45 93.98) (width 0.7) (layer B.Cu) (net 2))
 (segment (start 173.99 82.55) (end 173.99 91.44) (width 0.7) (layer B.Cu) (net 2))
 (segment (start 171.45 82.55) (end 173.99 82.55) (width 0.7) (layer B.Cu) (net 2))
 (segment (start 170.18 80.01) (end 170.18 81.28) (width 0.7) (layer B.Cu) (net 2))
 (segment (start 170.18 81.28) (end 171.45 82.55) (width 0.7) (layer B.Cu) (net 2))
 (segment (start 199.898 114.046) (end 202.946 114.046) (width 0.7) (layer B.Cu) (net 2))
 (segment (start 202.946 114.046) (end 204.47 112.522) (width 0.7) (layer B.Cu) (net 2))
 (segment (start 204.47 112.522) (end 204.47 67.31) (width 0.7) (layer B.Cu) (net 2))
 (segment (start 204.47 67.31) (end 168.91 67.31) (width 0.7) (layer B.Cu) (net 2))
 (segment (start 168.91 67.31) (end 168.91 76.2) (width 0.7) (layer B.Cu) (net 2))
 (segment (start 168.91 76.2) (end 170.18 77.47) (width 0.7) (layer B.Cu) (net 2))
 (segment (start 170.18 77.47) (end 170.18 80.01) (width 0.7) (layer B.Cu) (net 2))
 (segment (start 124.46 96.52) (end 130.81 96.52) (width 0.7) (layer B.Cu) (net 2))
 (segment (start 124.46 113.03) (end 124.46 96.52) (width 0.7) (layer B.Cu) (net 2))
 (segment (start 143.51 113.03) (end 124.46 113.03) (width 0.7) (layer B.Cu) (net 2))
 (segment (start 144.018 119.126) (end 144.018 113.538) (width 0.7) (layer B.Cu) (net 2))
 (segment (start 144.018 113.538) (end 143.51 113.03) (width 0.7) (layer B.Cu) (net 2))
 (segment (start 144.018 119.126) (end 146.558 119.126) (width 0.7) (layer B.Cu) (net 2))
 (segment (start 197.358 114.046) (end 199.898 114.046) (width 0.7) (layer B.Cu) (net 2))
 (segment (start 171.45 93.98) (end 133.35 93.98) (width 0.7) (layer B.Cu) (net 2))
 (segment (start 133.35 93.98) (end 130.81 96.52) (width 0.7) (layer B.Cu) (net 2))
 (segment (start 129.794 93.954) (end 129.794 70.866) (width 0.7) (layer B.Cu) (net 2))
 (segment (start 130.81 96.52) (end 130.81 94.97) (width 0.7) (layer B.Cu) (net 2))
 (segment (start 130.81 94.97) (end 129.794 93.954) (width 0.7) (layer B.Cu) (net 2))
 (segment (start 197.358 70.892) (end 197.358 70.866) (width 0.7) (layer F.Cu) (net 1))
 (segment (start 138.0744 115.57) (end 141.478 118.9736) (width 0.4) (layer B.Cu) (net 1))
 (segment (start 120.65 114.3) (end 121.92 115.57) (width 0.4) (layer B.Cu) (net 1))
 (segment (start 120.65 80.01) (end 120.65 114.3) (width 0.4) (layer B.Cu) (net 1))
 (segment (start 128.60539 72.05461) (end 120.65 80.01) (width 0.4) (layer B.Cu) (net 1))
 (segment (start 130.98261 73.83261) (end 130.98261 70.221262) (width 0.4) (layer B.Cu) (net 1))
 (segment (start 130.98261 70.221262) (end 130.286338 69.52499) (width 0.3) (layer B.Cu) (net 1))
 (segment (start 121.92 115.57) (end 138.0744 115.57) (width 0.4) (layer B.Cu) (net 1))
 (segment (start 130.286338 69.52499) (end 129.301662 69.52499) (width 0.3) (layer B.Cu) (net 1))
 (segment (start 141.478 118.9736) (end 141.478 119.126) (width 0.25) (layer B.Cu) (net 1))
 (segment (start 128.60539 70.221262) (end 128.60539 72.05461) (width 0.3) (layer B.Cu) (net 1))
 (segment (start 137.16 80.01) (end 130.98261 73.83261) (width 0.4) (layer B.Cu) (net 1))
 (segment (start 129.301662 69.52499) (end 128.60539 70.221262) (width 0.3) (layer B.Cu) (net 1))
 (segment (start 178.95 80.01) (end 177.8 80.01) (width 0.3) (layer B.Cu) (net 1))
 (segment (start 185.87161 73.08839) (end 178.95 80.01) (width 0.3) (layer B.Cu) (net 1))
 (segment (start 185.87161 70.323687) (end 185.87161 73.08839) (width 0.3) (layer B.Cu) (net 1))
 (segment (start 188.185287 68.01001) (end 185.87161 70.323687) (width 0.3) (layer B.Cu) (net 1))
 (segment (start 197.04201 68.01001) (end 188.185287 68.01001) (width 0.3) (layer B.Cu) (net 1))
 (segment (start 199.898 70.866) (end 197.04201 68.01001) (width 0.3) (layer B.Cu) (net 1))
 (segment (start 182.88 83.82) (end 182.88 96.52) (width 0.7) (layer B.Cu) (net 1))
 (segment (start 177.8 80.01) (end 177.8 83.82) (width 0.7) (layer B.Cu) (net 1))
 (segment (start 177.8 83.82) (end 182.88 83.82) (width 0.7) (layer B.Cu) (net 1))
 (segment (start 182.88 96.52) (end 171.45 96.52) (width 0.7) (layer B.Cu) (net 1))
 (segment (start 130.81 104.14) (end 151.13 104.14) (width 0.4) (layer B.Cu) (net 1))
 (segment (start 151.13 104.14) (end 151.13 119.38) (width 0.4) (layer B.Cu) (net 1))
 (segment (start 141.478 119.2784) (end 141.478 119.126) (width 0.4) (layer B.Cu) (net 1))
 (segment (start 149.96799 120.54201) (end 142.74161 120.54201) (width 0.4) (layer B.Cu) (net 1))
 (segment (start 142.74161 120.54201) (end 141.478 119.2784) (width 0.4) (layer B.Cu) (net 1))
 (segment (start 151.13 119.38) (end 149.96799 120.54201) (width 0.4) (layer B.Cu) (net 1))
 (segment (start 170.085001 97.884999) (end 128.175001 97.884999) (width 0.25) (layer B.Cu) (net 1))
 (segment (start 171.45 96.52) (end 170.085001 97.884999) (width 0.25) (layer B.Cu) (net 1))
 (segment (start 128.175001 97.884999) (end 128.27 97.979998) (width 0.25) (layer B.Cu) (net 1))
 (segment (start 128.27 101.6) (end 130.81 104.14) (width 0.25) (layer B.Cu) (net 1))
 (segment (start 128.27 97.979998) (end 128.27 101.6) (width 0.25) (layer B.Cu) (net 1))
 (segment (start 121.92 71.12) (end 122.174 70.866) (width 0.7) (layer F.Cu) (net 68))
 (segment (start 124.46 71.12) (end 124.714 70.866) (width 0.7) (layer F.Cu) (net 69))
 (segment (start 137.414 71.0184) (end 137.414 70.866) (width 0.7) (layer F.Cu) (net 14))
 (segment (start 139.7 80.01) (end 139.7 74.93) (width 0.7) (layer B.Cu) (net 14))
 (segment (start 137.414 72.644) (end 137.414 70.866) (width 0.7) (layer B.Cu) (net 14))
 (segment (start 139.7 74.93) (end 137.414 72.644) (width 0.7) (layer B.Cu) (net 14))
 (segment (start 139.954 71.0184) (end 139.954 70.866) (width 0.7) (layer F.Cu) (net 13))
 (segment (start 139.954 71.0184) (end 139.954 70.866) (width 0.7) (layer B.Cu) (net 13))
 (segment (start 142.24 73.3044) (end 139.954 71.0184) (width 0.7) (layer B.Cu) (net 13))
 (segment (start 142.24 80.01) (end 142.24 73.3044) (width 0.7) (layer B.Cu) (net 13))
 (segment (start 142.494 71.0184) (end 142.494 70.866) (width 0.7) (layer F.Cu) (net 12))
 (segment (start 142.494 71.0184) (end 142.494 70.866) (width 0.7) (layer B.Cu) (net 12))
 (segment (start 144.78 73.3044) (end 142.494 71.0184) (width 0.7) (layer B.Cu) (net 12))
 (segment (start 144.78 80.01) (end 144.78 73.3044) (width 0.7) (layer B.Cu) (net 12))
 (segment (start 145.796 70.866) (end 145.034 70.866) (width 0.7) (layer B.Cu) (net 11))
 (segment (start 147.32 80.01) (end 147.32 72.39) (width 0.7) (layer B.Cu) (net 11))
 (segment (start 147.32 72.39) (end 145.796 70.866) (width 0.7) (layer B.Cu) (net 11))
 (segment (start 149.86 71.628) (end 149.098 70.866) (width 0.7) (layer B.Cu) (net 10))
 (segment (start 149.86 80.01) (end 149.86 71.628) (width 0.7) (layer B.Cu) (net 10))
 (segment (start 152.4 71.628) (end 151.638 70.866) (width 0.7) (layer B.Cu) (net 9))
 (segment (start 152.4 80.01) (end 152.4 71.628) (width 0.7) (layer B.Cu) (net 9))
 (segment (start 154.94 71.628) (end 154.178 70.866) (width 0.7) (layer B.Cu) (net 8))
 (segment (start 154.94 80.01) (end 154.94 71.628) (width 0.7) (layer B.Cu) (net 8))
 (segment (start 157.48 71.628) (end 156.718 70.866) (width 0.7) (layer B.Cu) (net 7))
 (segment (start 157.48 80.01) (end 157.48 71.628) (width 0.7) (layer B.Cu) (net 7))
 (segment (start 171.45 99.06) (end 186.69 99.06) (width 0.7) (layer B.Cu) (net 3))
 (segment (start 187.198 98.552) (end 186.69 99.06) (width 0.7) (layer B.Cu) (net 3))
 (segment (start 187.198 70.866) (end 187.198 98.552) (width 0.7) (layer B.Cu) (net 3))
 (segment (start 140.97 99.06) (end 130.81 99.06) (width 0.7) (layer B.Cu) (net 3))
 (segment (start 171.45 99.06) (end 140.97 99.06) (width 0.7) (layer B.Cu) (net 3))
 (segment (start 189.738 70.866) (end 189.738 101.092) (width 0.7) (layer B.Cu) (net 4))
 (segment (start 189.23 101.6) (end 171.45 101.6) (width 0.7) (layer B.Cu) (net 4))
 (segment (start 189.738 101.092) (end 189.23 101.6) (width 0.7) (layer B.Cu) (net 4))
 (segment (start 171.45 101.6) (end 130.81 101.6) (width 0.7) (layer B.Cu) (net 4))
 (segment (start 182.118 71.0184) (end 182.118 70.866) (width 0.7) (layer F.Cu) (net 5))
 (segment (start 172.72 74.93) (end 172.72 80.01) (width 0.7) (layer B.Cu) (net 5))
 (segment (start 173.99 73.66) (end 172.72 74.93) (width 0.7) (layer B.Cu) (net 5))
 (segment (start 179.4764 73.66) (end 173.99 73.66) (width 0.7) (layer B.Cu) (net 5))
 (segment (start 182.118 70.866) (end 182.118 71.0184) (width 0.7) (layer B.Cu) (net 5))
 (segment (start 182.118 71.0184) (end 179.4764 73.66) (width 0.7) (layer B.Cu) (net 5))
 (segment (start 184.658 70.866) (end 184.658 71.0184) (width 0.7) (layer F.Cu) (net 6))
 (segment (start 179.4764 76.2) (end 175.26 76.2) (width 0.7) (layer B.Cu) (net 6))
 (segment (start 184.658 71.0184) (end 179.4764 76.2) (width 0.7) (layer B.Cu) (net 6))
 (segment (start 184.658 70.866) (end 184.658 71.0184) (width 0.7) (layer B.Cu) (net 6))
 (segment (start 175.26 80.01) (end 175.26 76.2) (width 0.7) (layer B.Cu) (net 6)))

